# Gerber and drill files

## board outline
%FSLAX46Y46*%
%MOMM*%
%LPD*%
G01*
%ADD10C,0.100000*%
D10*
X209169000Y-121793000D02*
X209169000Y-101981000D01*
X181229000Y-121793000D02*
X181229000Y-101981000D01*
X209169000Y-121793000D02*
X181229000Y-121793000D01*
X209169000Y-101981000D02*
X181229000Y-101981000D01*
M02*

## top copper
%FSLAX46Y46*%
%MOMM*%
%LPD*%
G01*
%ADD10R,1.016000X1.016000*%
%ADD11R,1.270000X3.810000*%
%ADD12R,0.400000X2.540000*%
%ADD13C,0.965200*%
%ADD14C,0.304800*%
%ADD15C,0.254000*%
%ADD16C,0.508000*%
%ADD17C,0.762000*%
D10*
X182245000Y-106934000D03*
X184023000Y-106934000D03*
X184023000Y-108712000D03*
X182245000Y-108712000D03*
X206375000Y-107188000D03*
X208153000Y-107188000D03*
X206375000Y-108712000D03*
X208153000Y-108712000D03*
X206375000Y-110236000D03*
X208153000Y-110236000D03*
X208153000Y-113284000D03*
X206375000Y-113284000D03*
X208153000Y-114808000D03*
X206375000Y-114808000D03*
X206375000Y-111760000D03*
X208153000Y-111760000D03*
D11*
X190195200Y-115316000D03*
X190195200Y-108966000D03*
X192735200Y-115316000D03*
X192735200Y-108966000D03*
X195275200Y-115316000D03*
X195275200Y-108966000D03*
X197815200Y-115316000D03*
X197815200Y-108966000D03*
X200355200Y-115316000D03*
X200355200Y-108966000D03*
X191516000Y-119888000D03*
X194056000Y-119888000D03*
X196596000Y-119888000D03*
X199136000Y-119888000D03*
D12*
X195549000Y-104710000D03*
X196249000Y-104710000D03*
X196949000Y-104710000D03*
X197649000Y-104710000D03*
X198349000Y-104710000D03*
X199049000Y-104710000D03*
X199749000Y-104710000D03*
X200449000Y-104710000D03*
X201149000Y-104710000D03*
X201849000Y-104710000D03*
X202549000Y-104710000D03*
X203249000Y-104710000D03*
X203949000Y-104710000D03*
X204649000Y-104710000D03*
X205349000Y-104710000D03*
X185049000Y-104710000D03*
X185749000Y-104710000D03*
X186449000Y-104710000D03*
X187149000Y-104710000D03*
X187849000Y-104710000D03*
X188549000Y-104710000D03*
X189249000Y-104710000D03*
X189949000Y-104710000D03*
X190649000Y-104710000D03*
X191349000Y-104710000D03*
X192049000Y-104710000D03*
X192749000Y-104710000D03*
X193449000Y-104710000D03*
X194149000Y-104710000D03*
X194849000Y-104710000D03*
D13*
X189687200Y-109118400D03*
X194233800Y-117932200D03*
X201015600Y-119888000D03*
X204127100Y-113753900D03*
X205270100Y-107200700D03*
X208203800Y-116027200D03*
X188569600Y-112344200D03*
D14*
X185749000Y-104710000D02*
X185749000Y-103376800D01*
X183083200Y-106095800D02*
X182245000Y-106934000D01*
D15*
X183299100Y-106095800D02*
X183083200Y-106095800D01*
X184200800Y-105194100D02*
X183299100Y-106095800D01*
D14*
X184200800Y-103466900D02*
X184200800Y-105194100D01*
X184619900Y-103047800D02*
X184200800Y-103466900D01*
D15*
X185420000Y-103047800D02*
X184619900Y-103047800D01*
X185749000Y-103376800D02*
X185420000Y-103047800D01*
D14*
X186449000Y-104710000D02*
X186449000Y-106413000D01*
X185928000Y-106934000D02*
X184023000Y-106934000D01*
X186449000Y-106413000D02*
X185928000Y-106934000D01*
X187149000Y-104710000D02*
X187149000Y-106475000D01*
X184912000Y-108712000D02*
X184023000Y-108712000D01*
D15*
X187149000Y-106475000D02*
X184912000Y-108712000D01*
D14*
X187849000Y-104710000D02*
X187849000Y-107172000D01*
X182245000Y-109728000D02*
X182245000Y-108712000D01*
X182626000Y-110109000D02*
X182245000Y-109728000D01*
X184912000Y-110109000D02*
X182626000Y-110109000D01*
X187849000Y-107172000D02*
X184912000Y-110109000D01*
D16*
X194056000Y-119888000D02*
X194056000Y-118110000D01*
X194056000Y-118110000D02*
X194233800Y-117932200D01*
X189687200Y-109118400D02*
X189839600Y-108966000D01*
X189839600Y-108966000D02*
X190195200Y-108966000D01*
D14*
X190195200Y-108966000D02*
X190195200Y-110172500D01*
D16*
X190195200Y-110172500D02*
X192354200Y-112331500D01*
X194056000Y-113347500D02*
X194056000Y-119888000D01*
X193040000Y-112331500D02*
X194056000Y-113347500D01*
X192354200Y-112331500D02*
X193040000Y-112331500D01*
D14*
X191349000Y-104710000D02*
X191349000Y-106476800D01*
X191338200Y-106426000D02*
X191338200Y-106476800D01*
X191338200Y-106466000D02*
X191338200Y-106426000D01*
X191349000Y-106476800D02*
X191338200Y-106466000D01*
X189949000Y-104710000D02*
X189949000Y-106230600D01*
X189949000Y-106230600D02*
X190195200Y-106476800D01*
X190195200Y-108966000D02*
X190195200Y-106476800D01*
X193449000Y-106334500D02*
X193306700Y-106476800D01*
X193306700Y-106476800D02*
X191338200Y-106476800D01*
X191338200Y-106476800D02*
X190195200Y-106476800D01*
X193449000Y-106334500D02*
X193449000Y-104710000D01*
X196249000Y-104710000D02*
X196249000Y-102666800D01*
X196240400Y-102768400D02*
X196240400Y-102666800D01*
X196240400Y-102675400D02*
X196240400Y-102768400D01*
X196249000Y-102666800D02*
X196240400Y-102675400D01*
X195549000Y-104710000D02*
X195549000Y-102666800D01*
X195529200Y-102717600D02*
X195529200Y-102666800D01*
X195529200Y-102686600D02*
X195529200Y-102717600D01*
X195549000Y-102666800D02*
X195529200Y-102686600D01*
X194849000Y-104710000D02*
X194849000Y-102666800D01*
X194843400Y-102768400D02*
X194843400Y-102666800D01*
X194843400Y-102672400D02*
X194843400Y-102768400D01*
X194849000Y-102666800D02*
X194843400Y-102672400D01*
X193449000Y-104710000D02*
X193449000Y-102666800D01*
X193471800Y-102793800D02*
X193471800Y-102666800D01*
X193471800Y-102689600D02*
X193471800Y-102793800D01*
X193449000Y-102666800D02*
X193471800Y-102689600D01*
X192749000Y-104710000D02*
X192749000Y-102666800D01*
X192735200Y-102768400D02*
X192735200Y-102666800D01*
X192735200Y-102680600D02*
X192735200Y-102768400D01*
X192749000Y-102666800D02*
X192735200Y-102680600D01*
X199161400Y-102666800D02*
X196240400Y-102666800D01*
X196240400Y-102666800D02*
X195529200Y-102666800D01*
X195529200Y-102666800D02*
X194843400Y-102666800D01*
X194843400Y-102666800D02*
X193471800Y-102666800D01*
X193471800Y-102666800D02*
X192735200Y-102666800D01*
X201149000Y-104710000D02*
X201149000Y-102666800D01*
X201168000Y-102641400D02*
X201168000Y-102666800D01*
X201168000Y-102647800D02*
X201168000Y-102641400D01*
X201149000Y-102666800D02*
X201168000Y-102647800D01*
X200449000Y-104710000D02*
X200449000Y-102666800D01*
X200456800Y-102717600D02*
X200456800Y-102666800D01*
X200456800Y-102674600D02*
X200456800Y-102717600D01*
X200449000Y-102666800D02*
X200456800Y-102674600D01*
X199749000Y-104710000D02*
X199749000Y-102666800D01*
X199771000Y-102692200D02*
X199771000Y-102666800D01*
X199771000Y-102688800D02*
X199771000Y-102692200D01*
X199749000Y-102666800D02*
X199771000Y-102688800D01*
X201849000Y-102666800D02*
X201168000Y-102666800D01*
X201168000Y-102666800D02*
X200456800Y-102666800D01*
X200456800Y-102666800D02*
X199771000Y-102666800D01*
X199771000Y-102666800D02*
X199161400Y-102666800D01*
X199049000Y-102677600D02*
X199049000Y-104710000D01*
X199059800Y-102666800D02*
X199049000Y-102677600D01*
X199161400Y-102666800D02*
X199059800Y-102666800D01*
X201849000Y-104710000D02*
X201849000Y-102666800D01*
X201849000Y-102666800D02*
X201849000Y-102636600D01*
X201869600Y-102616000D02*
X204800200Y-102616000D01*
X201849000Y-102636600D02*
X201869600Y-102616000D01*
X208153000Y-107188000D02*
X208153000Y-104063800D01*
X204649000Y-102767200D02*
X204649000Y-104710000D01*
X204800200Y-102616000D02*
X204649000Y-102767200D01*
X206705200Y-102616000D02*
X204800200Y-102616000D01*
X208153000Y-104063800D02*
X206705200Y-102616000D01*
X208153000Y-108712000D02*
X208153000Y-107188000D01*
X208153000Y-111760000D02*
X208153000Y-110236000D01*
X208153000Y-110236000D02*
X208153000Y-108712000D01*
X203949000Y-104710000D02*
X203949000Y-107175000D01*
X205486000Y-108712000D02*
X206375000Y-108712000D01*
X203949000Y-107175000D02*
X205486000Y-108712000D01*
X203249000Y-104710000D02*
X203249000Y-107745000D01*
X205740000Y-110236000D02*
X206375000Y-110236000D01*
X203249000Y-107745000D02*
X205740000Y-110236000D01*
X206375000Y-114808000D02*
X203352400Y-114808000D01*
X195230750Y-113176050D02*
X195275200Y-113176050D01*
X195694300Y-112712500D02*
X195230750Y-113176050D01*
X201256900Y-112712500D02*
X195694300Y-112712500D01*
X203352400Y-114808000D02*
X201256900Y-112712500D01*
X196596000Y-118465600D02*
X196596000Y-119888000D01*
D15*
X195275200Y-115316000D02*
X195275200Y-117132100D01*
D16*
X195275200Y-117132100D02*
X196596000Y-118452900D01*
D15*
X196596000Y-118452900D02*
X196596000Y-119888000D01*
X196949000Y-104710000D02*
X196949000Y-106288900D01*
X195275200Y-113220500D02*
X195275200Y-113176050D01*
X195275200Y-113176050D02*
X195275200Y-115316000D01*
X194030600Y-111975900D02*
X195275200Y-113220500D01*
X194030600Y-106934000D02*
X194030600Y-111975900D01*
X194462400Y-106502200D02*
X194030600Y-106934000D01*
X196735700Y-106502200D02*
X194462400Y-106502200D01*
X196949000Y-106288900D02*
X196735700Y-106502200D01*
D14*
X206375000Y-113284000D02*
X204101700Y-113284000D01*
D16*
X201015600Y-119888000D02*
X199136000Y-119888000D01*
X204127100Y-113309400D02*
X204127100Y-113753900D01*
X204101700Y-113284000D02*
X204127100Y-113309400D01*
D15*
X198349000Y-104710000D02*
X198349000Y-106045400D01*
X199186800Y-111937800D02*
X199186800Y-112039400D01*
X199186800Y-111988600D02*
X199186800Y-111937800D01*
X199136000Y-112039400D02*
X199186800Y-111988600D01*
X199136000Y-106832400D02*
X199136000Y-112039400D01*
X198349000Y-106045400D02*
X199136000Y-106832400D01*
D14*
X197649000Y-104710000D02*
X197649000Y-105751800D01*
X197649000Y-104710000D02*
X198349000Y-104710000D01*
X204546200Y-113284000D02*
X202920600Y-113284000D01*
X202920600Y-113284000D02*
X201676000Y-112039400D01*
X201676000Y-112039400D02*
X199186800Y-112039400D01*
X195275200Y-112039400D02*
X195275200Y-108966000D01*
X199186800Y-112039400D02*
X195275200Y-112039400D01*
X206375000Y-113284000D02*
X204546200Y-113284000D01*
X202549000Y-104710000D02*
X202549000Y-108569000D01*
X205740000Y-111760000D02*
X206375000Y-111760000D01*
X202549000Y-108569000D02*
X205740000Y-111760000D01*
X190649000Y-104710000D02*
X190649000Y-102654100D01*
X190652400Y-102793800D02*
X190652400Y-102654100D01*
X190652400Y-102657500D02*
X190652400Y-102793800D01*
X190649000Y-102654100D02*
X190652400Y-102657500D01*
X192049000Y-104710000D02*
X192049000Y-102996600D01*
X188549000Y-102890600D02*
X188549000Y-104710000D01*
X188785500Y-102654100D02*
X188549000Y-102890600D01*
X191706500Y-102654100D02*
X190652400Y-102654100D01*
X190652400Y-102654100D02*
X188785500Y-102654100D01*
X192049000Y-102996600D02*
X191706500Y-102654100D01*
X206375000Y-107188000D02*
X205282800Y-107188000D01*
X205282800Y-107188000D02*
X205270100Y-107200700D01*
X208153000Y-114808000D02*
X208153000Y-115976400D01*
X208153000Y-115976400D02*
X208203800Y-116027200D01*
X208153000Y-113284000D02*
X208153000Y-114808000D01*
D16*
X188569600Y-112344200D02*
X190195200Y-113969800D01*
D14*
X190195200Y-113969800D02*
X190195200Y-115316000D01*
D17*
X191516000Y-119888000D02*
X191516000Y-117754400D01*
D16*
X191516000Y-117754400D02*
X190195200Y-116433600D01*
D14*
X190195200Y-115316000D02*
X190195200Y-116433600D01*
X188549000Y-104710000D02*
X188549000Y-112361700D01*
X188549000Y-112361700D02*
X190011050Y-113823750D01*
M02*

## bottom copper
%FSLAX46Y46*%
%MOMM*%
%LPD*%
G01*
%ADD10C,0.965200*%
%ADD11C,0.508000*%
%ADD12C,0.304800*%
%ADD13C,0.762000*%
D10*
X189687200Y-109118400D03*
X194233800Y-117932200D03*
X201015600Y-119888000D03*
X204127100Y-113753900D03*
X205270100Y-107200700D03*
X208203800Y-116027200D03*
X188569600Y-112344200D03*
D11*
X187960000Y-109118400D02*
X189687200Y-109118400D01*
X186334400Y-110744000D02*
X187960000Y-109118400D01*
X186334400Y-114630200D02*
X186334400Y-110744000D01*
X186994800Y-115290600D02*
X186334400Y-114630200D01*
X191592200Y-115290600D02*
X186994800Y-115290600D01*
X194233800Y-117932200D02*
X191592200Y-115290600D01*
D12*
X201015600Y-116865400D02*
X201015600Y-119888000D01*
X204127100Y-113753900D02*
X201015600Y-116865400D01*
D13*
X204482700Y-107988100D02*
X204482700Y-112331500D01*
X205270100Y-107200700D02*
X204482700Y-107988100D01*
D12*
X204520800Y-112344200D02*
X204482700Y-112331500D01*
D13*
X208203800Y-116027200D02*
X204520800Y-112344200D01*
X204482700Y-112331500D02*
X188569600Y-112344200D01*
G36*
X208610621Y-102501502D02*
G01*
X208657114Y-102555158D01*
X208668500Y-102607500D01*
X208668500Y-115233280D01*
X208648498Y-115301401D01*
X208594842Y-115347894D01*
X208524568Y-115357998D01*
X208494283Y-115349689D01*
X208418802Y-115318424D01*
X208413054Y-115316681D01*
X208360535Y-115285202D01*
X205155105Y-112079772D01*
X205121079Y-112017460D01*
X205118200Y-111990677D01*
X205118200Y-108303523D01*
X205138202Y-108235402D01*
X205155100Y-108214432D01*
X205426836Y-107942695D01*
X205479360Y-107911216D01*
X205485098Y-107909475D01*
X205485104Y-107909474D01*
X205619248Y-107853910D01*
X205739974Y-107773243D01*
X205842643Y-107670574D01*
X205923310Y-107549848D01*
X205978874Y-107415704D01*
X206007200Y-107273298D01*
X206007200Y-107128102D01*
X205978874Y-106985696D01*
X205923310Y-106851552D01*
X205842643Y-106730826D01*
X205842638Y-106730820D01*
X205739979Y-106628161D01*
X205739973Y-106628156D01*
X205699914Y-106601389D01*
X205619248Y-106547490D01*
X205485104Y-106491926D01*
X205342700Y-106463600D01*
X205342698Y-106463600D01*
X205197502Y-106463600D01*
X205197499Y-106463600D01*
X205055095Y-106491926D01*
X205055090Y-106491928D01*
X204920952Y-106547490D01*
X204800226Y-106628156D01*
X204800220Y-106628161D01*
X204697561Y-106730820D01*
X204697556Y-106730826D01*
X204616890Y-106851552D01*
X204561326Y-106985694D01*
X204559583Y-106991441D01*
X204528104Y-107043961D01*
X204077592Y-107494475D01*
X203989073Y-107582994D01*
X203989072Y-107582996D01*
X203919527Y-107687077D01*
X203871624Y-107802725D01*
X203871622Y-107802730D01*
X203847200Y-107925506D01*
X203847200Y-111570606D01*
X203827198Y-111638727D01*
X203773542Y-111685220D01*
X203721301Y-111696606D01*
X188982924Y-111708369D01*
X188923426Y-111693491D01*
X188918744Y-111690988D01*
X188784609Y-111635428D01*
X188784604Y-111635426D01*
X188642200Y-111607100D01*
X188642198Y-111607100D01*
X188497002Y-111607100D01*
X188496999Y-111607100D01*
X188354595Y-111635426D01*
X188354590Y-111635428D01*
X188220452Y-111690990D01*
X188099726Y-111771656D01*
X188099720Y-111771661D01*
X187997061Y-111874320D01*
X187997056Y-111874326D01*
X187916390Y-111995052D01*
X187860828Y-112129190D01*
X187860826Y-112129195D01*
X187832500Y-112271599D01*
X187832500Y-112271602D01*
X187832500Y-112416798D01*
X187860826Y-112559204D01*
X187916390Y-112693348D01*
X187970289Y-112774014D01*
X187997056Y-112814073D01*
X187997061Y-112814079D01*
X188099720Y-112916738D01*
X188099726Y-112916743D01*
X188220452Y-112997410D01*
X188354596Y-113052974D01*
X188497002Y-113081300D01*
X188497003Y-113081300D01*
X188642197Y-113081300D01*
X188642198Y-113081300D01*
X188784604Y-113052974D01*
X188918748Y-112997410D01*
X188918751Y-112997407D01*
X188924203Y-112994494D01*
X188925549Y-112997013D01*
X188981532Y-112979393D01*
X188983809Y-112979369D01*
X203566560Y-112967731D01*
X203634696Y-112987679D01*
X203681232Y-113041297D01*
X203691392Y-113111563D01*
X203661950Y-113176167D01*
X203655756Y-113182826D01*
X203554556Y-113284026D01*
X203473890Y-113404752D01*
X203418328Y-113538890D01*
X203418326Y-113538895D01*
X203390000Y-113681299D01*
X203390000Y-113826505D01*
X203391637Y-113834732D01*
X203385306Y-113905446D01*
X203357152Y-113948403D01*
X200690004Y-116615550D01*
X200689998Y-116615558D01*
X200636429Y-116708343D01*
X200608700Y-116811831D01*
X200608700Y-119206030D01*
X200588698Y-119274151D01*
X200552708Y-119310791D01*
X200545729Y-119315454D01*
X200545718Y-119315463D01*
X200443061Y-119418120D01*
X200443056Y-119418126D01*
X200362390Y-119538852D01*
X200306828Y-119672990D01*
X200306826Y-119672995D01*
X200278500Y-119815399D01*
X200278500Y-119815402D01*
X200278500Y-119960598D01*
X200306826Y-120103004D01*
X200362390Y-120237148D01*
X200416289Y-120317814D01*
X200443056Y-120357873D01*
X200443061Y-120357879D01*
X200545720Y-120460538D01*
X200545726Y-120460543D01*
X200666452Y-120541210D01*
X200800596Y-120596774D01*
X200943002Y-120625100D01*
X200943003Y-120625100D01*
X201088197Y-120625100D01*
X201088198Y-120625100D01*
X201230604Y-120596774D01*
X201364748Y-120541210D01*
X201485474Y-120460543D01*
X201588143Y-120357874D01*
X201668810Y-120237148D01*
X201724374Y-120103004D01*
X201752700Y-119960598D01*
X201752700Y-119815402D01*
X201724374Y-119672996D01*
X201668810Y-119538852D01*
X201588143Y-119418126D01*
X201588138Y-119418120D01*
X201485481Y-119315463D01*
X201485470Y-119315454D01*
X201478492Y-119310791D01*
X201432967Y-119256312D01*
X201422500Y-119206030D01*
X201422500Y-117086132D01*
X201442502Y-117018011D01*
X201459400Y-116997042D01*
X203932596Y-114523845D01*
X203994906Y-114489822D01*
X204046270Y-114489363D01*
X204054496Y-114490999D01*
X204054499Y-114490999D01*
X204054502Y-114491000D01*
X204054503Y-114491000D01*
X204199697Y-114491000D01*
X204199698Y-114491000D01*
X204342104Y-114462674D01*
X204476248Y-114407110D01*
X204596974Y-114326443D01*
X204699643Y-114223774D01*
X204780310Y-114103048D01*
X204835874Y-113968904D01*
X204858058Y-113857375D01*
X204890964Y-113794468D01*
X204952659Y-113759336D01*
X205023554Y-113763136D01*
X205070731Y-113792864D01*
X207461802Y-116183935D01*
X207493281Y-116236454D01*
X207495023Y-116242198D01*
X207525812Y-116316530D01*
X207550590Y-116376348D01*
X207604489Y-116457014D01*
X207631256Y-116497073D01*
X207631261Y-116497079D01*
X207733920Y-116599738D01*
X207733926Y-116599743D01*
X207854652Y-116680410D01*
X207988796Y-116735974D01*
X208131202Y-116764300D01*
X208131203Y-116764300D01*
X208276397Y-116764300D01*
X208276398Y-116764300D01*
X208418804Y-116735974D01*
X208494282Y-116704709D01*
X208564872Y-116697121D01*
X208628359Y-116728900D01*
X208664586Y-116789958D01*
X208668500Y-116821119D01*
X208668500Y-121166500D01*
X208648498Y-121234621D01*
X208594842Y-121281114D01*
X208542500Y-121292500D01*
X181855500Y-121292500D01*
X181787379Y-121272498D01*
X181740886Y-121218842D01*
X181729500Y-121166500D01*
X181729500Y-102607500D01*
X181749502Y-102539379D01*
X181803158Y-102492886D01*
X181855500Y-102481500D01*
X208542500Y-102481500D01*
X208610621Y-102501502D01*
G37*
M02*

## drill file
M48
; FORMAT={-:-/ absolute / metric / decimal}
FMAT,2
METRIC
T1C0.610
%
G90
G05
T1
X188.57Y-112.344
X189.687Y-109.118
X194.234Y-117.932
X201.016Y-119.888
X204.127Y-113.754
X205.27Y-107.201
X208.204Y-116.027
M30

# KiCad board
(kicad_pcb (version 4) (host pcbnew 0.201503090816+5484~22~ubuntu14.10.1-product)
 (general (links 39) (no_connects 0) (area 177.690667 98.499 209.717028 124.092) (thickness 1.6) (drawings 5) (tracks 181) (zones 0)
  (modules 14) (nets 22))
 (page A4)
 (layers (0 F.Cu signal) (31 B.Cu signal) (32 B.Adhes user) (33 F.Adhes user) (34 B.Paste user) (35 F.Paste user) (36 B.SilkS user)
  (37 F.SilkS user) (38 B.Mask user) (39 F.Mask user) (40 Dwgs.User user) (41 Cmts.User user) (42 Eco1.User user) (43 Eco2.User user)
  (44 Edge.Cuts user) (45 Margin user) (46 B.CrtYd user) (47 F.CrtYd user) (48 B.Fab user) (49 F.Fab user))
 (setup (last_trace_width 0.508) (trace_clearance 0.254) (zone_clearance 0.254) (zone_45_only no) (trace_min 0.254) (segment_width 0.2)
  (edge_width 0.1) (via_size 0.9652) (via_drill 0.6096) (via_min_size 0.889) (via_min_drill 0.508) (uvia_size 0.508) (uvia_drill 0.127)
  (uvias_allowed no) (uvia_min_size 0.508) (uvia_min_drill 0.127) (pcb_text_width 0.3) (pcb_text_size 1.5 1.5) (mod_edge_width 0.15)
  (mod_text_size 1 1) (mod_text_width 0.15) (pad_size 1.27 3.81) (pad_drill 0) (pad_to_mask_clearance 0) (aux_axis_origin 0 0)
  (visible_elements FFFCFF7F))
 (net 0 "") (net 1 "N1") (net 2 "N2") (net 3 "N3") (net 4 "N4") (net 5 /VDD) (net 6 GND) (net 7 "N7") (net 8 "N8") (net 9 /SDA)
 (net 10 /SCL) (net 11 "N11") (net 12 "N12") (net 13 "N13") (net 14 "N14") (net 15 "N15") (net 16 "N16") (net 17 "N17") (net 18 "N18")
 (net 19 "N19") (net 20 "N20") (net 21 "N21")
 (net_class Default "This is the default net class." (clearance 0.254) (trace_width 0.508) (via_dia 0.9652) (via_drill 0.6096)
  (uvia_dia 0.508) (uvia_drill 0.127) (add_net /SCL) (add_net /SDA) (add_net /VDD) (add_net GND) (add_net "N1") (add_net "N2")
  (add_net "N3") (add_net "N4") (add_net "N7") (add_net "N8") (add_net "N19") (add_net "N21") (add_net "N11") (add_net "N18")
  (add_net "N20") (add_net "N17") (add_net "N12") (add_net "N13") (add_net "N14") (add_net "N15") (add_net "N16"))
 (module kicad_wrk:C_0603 (layer F.Cu) (at 183.134 106.934)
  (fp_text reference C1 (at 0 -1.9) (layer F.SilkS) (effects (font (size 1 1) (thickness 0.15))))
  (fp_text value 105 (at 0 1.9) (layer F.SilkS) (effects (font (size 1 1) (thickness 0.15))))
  (pad 1 smd rect (at -0.889 0) (size 1.016 1.016) (layers F.Cu F.Paste F.Mask) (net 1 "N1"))
  (pad 2 smd rect (at 0.889 0) (size 1.016 1.016) (layers F.Cu F.Paste F.Mask) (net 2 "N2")))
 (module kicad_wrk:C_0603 (layer F.Cu) (at 183.134 108.712 180)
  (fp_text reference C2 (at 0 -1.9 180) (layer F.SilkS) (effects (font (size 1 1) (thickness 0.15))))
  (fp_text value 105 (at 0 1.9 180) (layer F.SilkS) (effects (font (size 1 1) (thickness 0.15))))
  (pad 1 smd rect (at -0.889 0 180) (size 1.016 1.016) (layers F.Cu F.Paste F.Mask) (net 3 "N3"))
  (pad 2 smd rect (at 0.889 0 180) (size 1.016 1.016) (layers F.Cu F.Paste F.Mask) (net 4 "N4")))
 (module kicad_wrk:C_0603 (layer F.Cu) (at 207.264 107.188)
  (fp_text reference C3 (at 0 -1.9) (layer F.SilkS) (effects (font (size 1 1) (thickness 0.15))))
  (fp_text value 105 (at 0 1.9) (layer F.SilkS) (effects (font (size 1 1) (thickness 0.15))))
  (pad 1 smd rect (at -0.889 0) (size 1.016 1.016) (layers F.Cu F.Paste F.Mask) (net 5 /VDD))
  (pad 2 smd rect (at 0.889 0) (size 1.016 1.016) (layers F.Cu F.Paste F.Mask) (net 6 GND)))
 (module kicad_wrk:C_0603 (layer F.Cu) (at 207.264 108.712)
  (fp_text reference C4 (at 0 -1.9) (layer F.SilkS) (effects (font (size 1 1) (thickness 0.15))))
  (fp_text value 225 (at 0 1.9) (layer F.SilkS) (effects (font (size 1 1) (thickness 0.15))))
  (pad 1 smd rect (at -0.889 0) (size 1.016 1.016) (layers F.Cu F.Paste F.Mask) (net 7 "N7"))
  (pad 2 smd rect (at 0.889 0) (size 1.016 1.016) (layers F.Cu F.Paste F.Mask) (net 6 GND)))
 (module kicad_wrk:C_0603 (layer F.Cu) (at 207.264 110.236)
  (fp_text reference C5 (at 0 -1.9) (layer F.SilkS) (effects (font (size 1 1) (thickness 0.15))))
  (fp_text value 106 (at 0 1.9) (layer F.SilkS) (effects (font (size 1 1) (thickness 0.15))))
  (pad 1 smd rect (at -0.889 0) (size 1.016 1.016) (layers F.Cu F.Paste F.Mask) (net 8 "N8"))
  (pad 2 smd rect (at 0.889 0) (size 1.016 1.016) (layers F.Cu F.Paste F.Mask) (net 6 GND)))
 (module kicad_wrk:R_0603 (layer F.Cu) (at 207.264 113.284 180)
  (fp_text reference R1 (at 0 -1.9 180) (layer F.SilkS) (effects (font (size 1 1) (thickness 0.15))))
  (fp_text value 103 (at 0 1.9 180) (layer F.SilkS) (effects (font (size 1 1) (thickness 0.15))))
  (pad 1 smd rect (at -0.889 0 180) (size 1.016 1.016) (layers F.Cu F.Paste F.Mask) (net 5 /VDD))
  (pad 2 smd rect (at 0.889 0 180) (size 1.016 1.016) (layers F.Cu F.Paste F.Mask) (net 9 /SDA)))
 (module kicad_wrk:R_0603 (layer F.Cu) (at 207.264 114.808 180)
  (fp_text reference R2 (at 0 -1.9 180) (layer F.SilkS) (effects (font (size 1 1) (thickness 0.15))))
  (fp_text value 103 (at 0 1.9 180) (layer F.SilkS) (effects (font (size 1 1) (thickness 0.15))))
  (pad 1 smd rect (at -0.889 0 180) (size 1.016 1.016) (layers F.Cu F.Paste F.Mask) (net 5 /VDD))
  (pad 2 smd rect (at 0.889 0 180) (size 1.016 1.016) (layers F.Cu F.Paste F.Mask) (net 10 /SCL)))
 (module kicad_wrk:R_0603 (layer F.Cu) (at 207.264 111.76)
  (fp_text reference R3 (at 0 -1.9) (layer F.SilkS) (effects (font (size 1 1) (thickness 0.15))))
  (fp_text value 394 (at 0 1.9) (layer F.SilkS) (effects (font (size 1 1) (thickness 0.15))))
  (pad 1 smd rect (at -0.889 0) (size 1.016 1.016) (layers F.Cu F.Paste F.Mask) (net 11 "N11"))
  (pad 2 smd rect (at 0.889 0) (size 1.016 1.016) (layers F.Cu F.Paste F.Mask) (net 6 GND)))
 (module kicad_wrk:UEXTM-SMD (layer F.Cu) (at 195.2752 112.141 180)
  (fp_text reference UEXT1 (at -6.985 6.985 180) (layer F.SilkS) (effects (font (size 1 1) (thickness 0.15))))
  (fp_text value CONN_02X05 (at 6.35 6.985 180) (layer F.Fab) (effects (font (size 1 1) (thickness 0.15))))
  (pad 1 smd rect (at 5.08 -3.175 180) (size 1.27 3.81) (layers F.Cu F.Paste F.Mask) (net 5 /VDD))
  (pad 2 smd rect (at 5.08 3.175 180) (size 1.27 3.81) (layers F.Cu F.Paste F.Mask) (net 6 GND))
  (pad 3 smd rect (at 2.54 -3.175 180) (size 1.27 3.81) (layers F.Cu F.Paste F.Mask) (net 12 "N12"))
  (pad 4 smd rect (at 2.54 3.175 180) (size 1.27 3.81) (layers F.Cu F.Paste F.Mask) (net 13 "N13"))
  (pad 5 smd rect (at 0 -3.175 180) (size 1.27 3.81) (layers F.Cu F.Paste F.Mask) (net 10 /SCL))
  (pad 6 smd rect (at 0 3.175 180) (size 1.27 3.81) (layers F.Cu F.Paste F.Mask) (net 9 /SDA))
  (pad 7 smd rect (at -2.54 -3.175 180) (size 1.27 3.81) (layers F.Cu F.Paste F.Mask) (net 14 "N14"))
  (pad 8 smd rect (at -2.54 3.175 180) (size 1.27 3.81) (layers F.Cu F.Paste F.Mask) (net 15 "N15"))
  (pad 9 smd rect (at -5.08 -3.175 180) (size 1.27 3.81) (layers F.Cu F.Paste F.Mask) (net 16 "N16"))
  (pad 10 smd rect (at -5.08 3.175 180) (size 1.27 3.81) (layers F.Cu F.Paste F.Mask) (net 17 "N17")))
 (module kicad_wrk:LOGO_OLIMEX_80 (layer F.Cu) (at 205.5876 118.6942)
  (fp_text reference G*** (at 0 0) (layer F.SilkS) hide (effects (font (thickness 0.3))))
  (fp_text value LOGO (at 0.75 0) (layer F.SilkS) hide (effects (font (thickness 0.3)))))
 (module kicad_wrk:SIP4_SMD (layer F.Cu) (at 195.326 119.888)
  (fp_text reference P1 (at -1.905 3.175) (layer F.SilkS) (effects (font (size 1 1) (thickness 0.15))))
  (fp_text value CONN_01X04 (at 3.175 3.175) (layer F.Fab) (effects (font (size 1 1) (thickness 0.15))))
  (pad 1 smd rect (at -3.81 0) (size 1.27 3.81) (layers F.Cu F.Mask) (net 5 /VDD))
  (pad 2 smd rect (at -1.27 0) (size 1.27 3.81) (layers F.Cu F.Mask) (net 6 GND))
  (pad 3 smd rect (at 1.27 0) (size 1.27 3.81) (layers F.Cu F.Mask) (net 10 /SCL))
  (pad 4 smd rect (at 3.81 0) (size 1.27 3.81) (layers F.Cu F.Mask) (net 9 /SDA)))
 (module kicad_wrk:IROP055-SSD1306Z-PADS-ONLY (layer F.Cu) (at 195.199 105.41)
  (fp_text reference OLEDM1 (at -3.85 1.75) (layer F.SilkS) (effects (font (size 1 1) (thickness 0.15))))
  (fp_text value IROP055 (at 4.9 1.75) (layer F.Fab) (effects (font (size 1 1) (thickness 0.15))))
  (pad 16 smd rect (at 0.35 -0.7) (size 0.4 2.54) (layers F.Cu F.Paste F.Mask) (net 6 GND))
  (pad 17 smd rect (at 1.05 -0.7) (size 0.4 2.54) (layers F.Cu F.Paste F.Mask) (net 6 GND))
  (pad 18 smd rect (at 1.75 -0.7) (size 0.4 2.54) (layers F.Cu F.Paste F.Mask) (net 10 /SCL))
  (pad 19 smd rect (at 2.45 -0.7) (size 0.4 2.54) (layers F.Cu F.Paste F.Mask) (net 9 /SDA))
  (pad 20 smd rect (at 3.15 -0.7) (size 0.4 2.54) (layers F.Cu F.Paste F.Mask) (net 9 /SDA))
  (pad 21 smd rect (at 3.85 -0.7) (size 0.4 2.54) (layers F.Cu F.Paste F.Mask) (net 6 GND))
  (pad 22 smd rect (at 4.55 -0.7) (size 0.4 2.54) (layers F.Cu F.Paste F.Mask) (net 6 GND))
  (pad 23 smd rect (at 5.25 -0.7) (size 0.4 2.54) (layers F.Cu F.Paste F.Mask) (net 6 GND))
  (pad 24 smd rect (at 5.95 -0.7) (size 0.4 2.54) (layers F.Cu F.Paste F.Mask) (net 6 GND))
  (pad 25 smd rect (at 6.65 -0.7) (size 0.4 2.54) (layers F.Cu F.Paste F.Mask) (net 6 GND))
  (pad 26 smd rect (at 7.35 -0.7) (size 0.4 2.54) (layers F.Cu F.Paste F.Mask) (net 11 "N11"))
  (pad 27 smd rect (at 8.05 -0.7) (size 0.4 2.54) (layers F.Cu F.Paste F.Mask) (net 8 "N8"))
  (pad 28 smd rect (at 8.75 -0.7) (size 0.4 2.54) (layers F.Cu F.Paste F.Mask) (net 7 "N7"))
  (pad 29 smd rect (at 9.45 -0.7) (size 0.4 2.54) (layers F.Cu F.Paste F.Mask) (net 6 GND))
  (pad 30 smd rect (at 10.15 -0.7) (size 0.4 2.54) (layers F.Cu F.Paste F.Mask) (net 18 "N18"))
  (pad 1 smd rect (at -10.15 -0.7) (size 0.4 2.54) (layers F.Cu F.Paste F.Mask) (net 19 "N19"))
  (pad 2 smd rect (at -9.45 -0.7) (size 0.4 2.54) (layers F.Cu F.Paste F.Mask) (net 1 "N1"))
  (pad 3 smd rect (at -8.75 -0.7) (size 0.4 2.54) (layers F.Cu F.Paste F.Mask) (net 2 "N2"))
  (pad 4 smd rect (at -8.05 -0.7) (size 0.4 2.54) (layers F.Cu F.Paste F.Mask) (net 3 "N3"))
  (pad 5 smd rect (at -7.35 -0.7) (size 0.4 2.54) (layers F.Cu F.Paste F.Mask) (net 4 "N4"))
  (pad 6 smd rect (at -6.65 -0.7) (size 0.4 2.54) (layers F.Cu F.Paste F.Mask) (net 5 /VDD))
  (pad 7 smd rect (at -5.95 -0.7) (size 0.4 2.54) (layers F.Cu F.Paste F.Mask) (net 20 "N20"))
  (pad 8 smd rect (at -5.25 -0.7) (size 0.4 2.54) (layers F.Cu F.Paste F.Mask) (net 6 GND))
  (pad 9 smd rect (at -4.55 -0.7) (size 0.4 2.54) (layers F.Cu F.Paste F.Mask) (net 5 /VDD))
  (pad 10 smd rect (at -3.85 -0.7) (size 0.4 2.54) (layers F.Cu F.Paste F.Mask) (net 6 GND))
  (pad 11 smd rect (at -3.15 -0.7) (size 0.4 2.54) (layers F.Cu F.Paste F.Mask) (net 5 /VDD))
  (pad 12 smd rect (at -2.45 -0.7) (size 0.4 2.54) (layers F.Cu F.Paste F.Mask) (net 6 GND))
  (pad 13 smd rect (at -1.75 -0.7) (size 0.4 2.54) (layers F.Cu F.Paste F.Mask) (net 6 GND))
  (pad 14 smd rect (at -1.05 -0.7) (size 0.4 2.54) (layers F.Cu F.Paste F.Mask) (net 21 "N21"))
  (pad 15 smd rect (at -0.35 -0.7) (size 0.4 2.54) (layers F.Cu F.Paste F.Mask) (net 6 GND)))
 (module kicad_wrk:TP (layer F.Cu) (at 182.753 103.378 180)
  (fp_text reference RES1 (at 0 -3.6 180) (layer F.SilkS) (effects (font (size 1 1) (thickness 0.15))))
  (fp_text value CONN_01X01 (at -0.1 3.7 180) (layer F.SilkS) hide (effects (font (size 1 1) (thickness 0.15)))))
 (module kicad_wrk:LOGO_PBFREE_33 (layer F.Cu) (at 183.6166 118.8466)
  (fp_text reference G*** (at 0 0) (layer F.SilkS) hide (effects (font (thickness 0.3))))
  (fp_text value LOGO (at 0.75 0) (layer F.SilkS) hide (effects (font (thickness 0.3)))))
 (gr_line (start 209.169 121.793) (end 209.169 101.981) (angle 90) (layer Edge.Cuts) (width 0.1))
 (gr_line (start 181.229 121.793) (end 181.229 101.981) (angle 90) (layer Edge.Cuts) (width 0.1))
 (gr_line (start 209.169 121.793) (end 181.229 121.793) (angle 90) (layer Edge.Cuts) (width 0.1))
 (gr_line (start 209.169 101.981) (end 181.229 101.981) (angle 90) (layer Edge.Cuts) (width 0.1))
 (segment (start 185.749 104.71) (end 185.749 103.3768) (width 0.3048) (layer F.Cu) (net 1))
 (segment (start 183.0832 106.0958) (end 182.245 106.934) (width 0.3048) (layer F.Cu) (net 1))
 (segment (start 183.2991 106.0958) (end 183.0832 106.0958) (width 0.254) (layer F.Cu) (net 1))
 (segment (start 184.2008 105.1941) (end 183.2991 106.0958) (width 0.254) (layer F.Cu) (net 1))
 (segment (start 184.2008 103.4669) (end 184.2008 105.1941) (width 0.3048) (layer F.Cu) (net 1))
 (segment (start 184.6199 103.0478) (end 184.2008 103.4669) (width 0.3048) (layer F.Cu) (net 1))
 (segment (start 185.42 103.0478) (end 184.6199 103.0478) (width 0.254) (layer F.Cu) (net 1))
 (segment (start 185.749 103.3768) (end 185.42 103.0478) (width 0.254) (layer F.Cu) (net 1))
 (segment (start 186.449 104.71) (end 186.449 106.413) (width 0.3048) (layer F.Cu) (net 2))
 (segment (start 185.928 106.934) (end 184.023 106.934) (width 0.3048) (layer F.Cu) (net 2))
 (segment (start 186.449 106.413) (end 185.928 106.934) (width 0.3048) (layer F.Cu) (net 2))
 (segment (start 187.149 104.71) (end 187.149 106.475) (width 0.3048) (layer F.Cu) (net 3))
 (segment (start 184.912 108.712) (end 184.023 108.712) (width 0.3048) (layer F.Cu) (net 3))
 (segment (start 187.149 106.475) (end 184.912 108.712) (width 0.254) (layer F.Cu) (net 3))
 (segment (start 187.849 104.71) (end 187.849 107.172) (width 0.3048) (layer F.Cu) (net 4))
 (segment (start 182.245 109.728) (end 182.245 108.712) (width 0.3048) (layer F.Cu) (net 4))
 (segment (start 182.626 110.109) (end 182.245 109.728) (width 0.3048) (layer F.Cu) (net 4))
 (segment (start 184.912 110.109) (end 182.626 110.109) (width 0.3048) (layer F.Cu) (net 4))
 (segment (start 187.849 107.172) (end 184.912 110.109) (width 0.3048) (layer F.Cu) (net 4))
 (segment (start 194.056 119.888) (end 194.056 118.11) (width 0.508) (layer F.Cu) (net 6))
 (segment (start 194.056 118.11) (end 194.2338 117.9322) (width 0.508) (layer F.Cu) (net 6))
 (segment (start 189.6872 109.1184) (end 189.8396 108.966) (width 0.508) (layer F.Cu) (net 6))
 (via (at 189.6872 109.1184) (size 0.9652) (layers F.Cu B.Cu) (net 6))
 (segment (start 187.96 109.1184) (end 189.6872 109.1184) (width 0.508) (layer B.Cu) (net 6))
 (segment (start 186.3344 110.744) (end 187.96 109.1184) (width 0.508) (layer B.Cu) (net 6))
 (segment (start 186.3344 114.6302) (end 186.3344 110.744) (width 0.508) (layer B.Cu) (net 6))
 (segment (start 186.9948 115.2906) (end 186.3344 114.6302) (width 0.508) (layer B.Cu) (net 6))
 (segment (start 191.5922 115.2906) (end 186.9948 115.2906) (width 0.508) (layer B.Cu) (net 6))
 (segment (start 194.2338 117.9322) (end 191.5922 115.2906) (width 0.508) (layer B.Cu) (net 6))
 (via (at 194.2338 117.9322) (size 0.9652) (layers F.Cu B.Cu) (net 6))
 (segment (start 189.8396 108.966) (end 190.1952 108.966) (width 0.508) (layer F.Cu) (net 6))
 (segment (start 190.1952 108.966) (end 190.1952 110.1725) (width 0.3048) (layer F.Cu) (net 6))
 (segment (start 190.1952 110.1725) (end 192.3542 112.3315) (width 0.508) (layer F.Cu) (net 6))
 (segment (start 194.056 113.3475) (end 194.056 119.888) (width 0.508) (layer F.Cu) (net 6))
 (segment (start 193.04 112.3315) (end 194.056 113.3475) (width 0.508) (layer F.Cu) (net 6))
 (segment (start 192.3542 112.3315) (end 193.04 112.3315) (width 0.508) (layer F.Cu) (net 6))
 (segment (start 191.349 104.71) (end 191.349 106.4768) (width 0.3048) (layer F.Cu) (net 6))
 (segment (start 191.3382 106.426) (end 191.3382 106.4768) (width 0.3048) (layer F.Cu) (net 6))
 (segment (start 191.3382 106.466) (end 191.3382 106.426) (width 0.3048) (layer F.Cu) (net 6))
 (segment (start 191.349 106.4768) (end 191.3382 106.466) (width 0.3048) (layer F.Cu) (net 6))
 (segment (start 189.949 104.71) (end 189.949 106.2306) (width 0.3048) (layer F.Cu) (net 6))
 (segment (start 189.949 106.2306) (end 190.1952 106.4768) (width 0.3048) (layer F.Cu) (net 6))
 (segment (start 190.1952 108.966) (end 190.1952 106.4768) (width 0.3048) (layer F.Cu) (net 6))
 (segment (start 193.449 106.3345) (end 193.3067 106.4768) (width 0.3048) (layer F.Cu) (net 6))
 (segment (start 193.3067 106.4768) (end 191.3382 106.4768) (width 0.3048) (layer F.Cu) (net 6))
 (segment (start 191.3382 106.4768) (end 190.1952 106.4768) (width 0.3048) (layer F.Cu) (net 6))
 (segment (start 193.449 106.3345) (end 193.449 104.71) (width 0.3048) (layer F.Cu) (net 6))
 (segment (start 196.249 104.71) (end 196.249 102.6668) (width 0.3048) (layer F.Cu) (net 6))
 (segment (start 196.2404 102.7684) (end 196.2404 102.6668) (width 0.3048) (layer F.Cu) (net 6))
 (segment (start 196.2404 102.6754) (end 196.2404 102.7684) (width 0.3048) (layer F.Cu) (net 6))
 (segment (start 196.249 102.6668) (end 196.2404 102.6754) (width 0.3048) (layer F.Cu) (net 6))
 (segment (start 195.549 104.71) (end 195.549 102.6668) (width 0.3048) (layer F.Cu) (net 6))
 (segment (start 195.5292 102.7176) (end 195.5292 102.6668) (width 0.3048) (layer F.Cu) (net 6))
 (segment (start 195.5292 102.6866) (end 195.5292 102.7176) (width 0.3048) (layer F.Cu) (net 6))
 (segment (start 195.549 102.6668) (end 195.5292 102.6866) (width 0.3048) (layer F.Cu) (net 6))
 (segment (start 194.849 104.71) (end 194.849 102.6668) (width 0.3048) (layer F.Cu) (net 6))
 (segment (start 194.8434 102.7684) (end 194.8434 102.6668) (width 0.3048) (layer F.Cu) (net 6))
 (segment (start 194.8434 102.6724) (end 194.8434 102.7684) (width 0.3048) (layer F.Cu) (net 6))
 (segment (start 194.849 102.6668) (end 194.8434 102.6724) (width 0.3048) (layer F.Cu) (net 6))
 (segment (start 193.449 104.71) (end 193.449 102.6668) (width 0.3048) (layer F.Cu) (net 6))
 (segment (start 193.4718 102.7938) (end 193.4718 102.6668) (width 0.3048) (layer F.Cu) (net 6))
 (segment (start 193.4718 102.6896) (end 193.4718 102.7938) (width 0.3048) (layer F.Cu) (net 6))
 (segment (start 193.449 102.6668) (end 193.4718 102.6896) (width 0.3048) (layer F.Cu) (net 6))
 (segment (start 192.749 104.71) (end 192.749 102.6668) (width 0.3048) (layer F.Cu) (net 6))
 (segment (start 192.7352 102.7684) (end 192.7352 102.6668) (width 0.3048) (layer F.Cu) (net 6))
 (segment (start 192.7352 102.6806) (end 192.7352 102.7684) (width 0.3048) (layer F.Cu) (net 6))
 (segment (start 192.749 102.6668) (end 192.7352 102.6806) (width 0.3048) (layer F.Cu) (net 6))
 (segment (start 199.1614 102.6668) (end 196.2404 102.6668) (width 0.3048) (layer F.Cu) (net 6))
 (segment (start 196.2404 102.6668) (end 195.5292 102.6668) (width 0.3048) (layer F.Cu) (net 6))
 (segment (start 195.5292 102.6668) (end 194.8434 102.6668) (width 0.3048) (layer F.Cu) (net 6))
 (segment (start 194.8434 102.6668) (end 193.4718 102.6668) (width 0.3048) (layer F.Cu) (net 6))
 (segment (start 193.4718 102.6668) (end 192.7352 102.6668) (width 0.3048) (layer F.Cu) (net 6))
 (segment (start 201.149 104.71) (end 201.149 102.6668) (width 0.3048) (layer F.Cu) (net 6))
 (segment (start 201.168 102.6414) (end 201.168 102.6668) (width 0.3048) (layer F.Cu) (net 6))
 (segment (start 201.168 102.6478) (end 201.168 102.6414) (width 0.3048) (layer F.Cu) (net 6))
 (segment (start 201.149 102.6668) (end 201.168 102.6478) (width 0.3048) (layer F.Cu) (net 6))
 (segment (start 200.449 104.71) (end 200.449 102.6668) (width 0.3048) (layer F.Cu) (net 6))
 (segment (start 200.4568 102.7176) (end 200.4568 102.6668) (width 0.3048) (layer F.Cu) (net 6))
 (segment (start 200.4568 102.6746) (end 200.4568 102.7176) (width 0.3048) (layer F.Cu) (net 6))
 (segment (start 200.449 102.6668) (end 200.4568 102.6746) (width 0.3048) (layer F.Cu) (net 6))
 (segment (start 199.749 104.71) (end 199.749 102.6668) (width 0.3048) (layer F.Cu) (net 6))
 (segment (start 199.771 102.6922) (end 199.771 102.6668) (width 0.3048) (layer F.Cu) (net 6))
 (segment (start 199.771 102.6888) (end 199.771 102.6922) (width 0.3048) (layer F.Cu) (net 6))
 (segment (start 199.749 102.6668) (end 199.771 102.6888) (width 0.3048) (layer F.Cu) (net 6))
 (segment (start 201.849 102.6668) (end 201.168 102.6668) (width 0.3048) (layer F.Cu) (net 6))
 (segment (start 201.168 102.6668) (end 200.4568 102.6668) (width 0.3048) (layer F.Cu) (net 6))
 (segment (start 200.4568 102.6668) (end 199.771 102.6668) (width 0.3048) (layer F.Cu) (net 6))
 (segment (start 199.771 102.6668) (end 199.1614 102.6668) (width 0.3048) (layer F.Cu) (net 6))
 (segment (start 199.049 102.6776) (end 199.049 104.71) (width 0.3048) (layer F.Cu) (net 6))
 (segment (start 199.0598 102.6668) (end 199.049 102.6776) (width 0.3048) (layer F.Cu) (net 6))
 (segment (start 199.1614 102.6668) (end 199.0598 102.6668) (width 0.3048) (layer F.Cu) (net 6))
 (segment (start 201.849 104.71) (end 201.849 102.6668) (width 0.3048) (layer F.Cu) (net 6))
 (segment (start 201.849 102.6668) (end 201.849 102.6366) (width 0.3048) (layer F.Cu) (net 6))
 (segment (start 201.8696 102.616) (end 204.8002 102.616) (width 0.3048) (layer F.Cu) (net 6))
 (segment (start 201.849 102.6366) (end 201.8696 102.616) (width 0.3048) (layer F.Cu) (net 6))
 (segment (start 208.153 107.188) (end 208.153 104.0638) (width 0.3048) (layer F.Cu) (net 6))
 (segment (start 204.649 102.7672) (end 204.649 104.71) (width 0.3048) (layer F.Cu) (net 6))
 (segment (start 204.8002 102.616) (end 204.649 102.7672) (width 0.3048) (layer F.Cu) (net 6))
 (segment (start 206.7052 102.616) (end 204.8002 102.616) (width 0.3048) (layer F.Cu) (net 6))
 (segment (start 208.153 104.0638) (end 206.7052 102.616) (width 0.3048) (layer F.Cu) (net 6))
 (segment (start 208.153 108.712) (end 208.153 107.188) (width 0.3048) (layer F.Cu) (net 6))
 (segment (start 208.153 111.76) (end 208.153 110.236) (width 0.3048) (layer F.Cu) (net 6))
 (segment (start 208.153 110.236) (end 208.153 108.712) (width 0.3048) (layer F.Cu) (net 6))
 (segment (start 203.949 104.71) (end 203.949 107.175) (width 0.3048) (layer F.Cu) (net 7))
 (segment (start 205.486 108.712) (end 206.375 108.712) (width 0.3048) (layer F.Cu) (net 7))
 (segment (start 203.949 107.175) (end 205.486 108.712) (width 0.3048) (layer F.Cu) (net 7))
 (segment (start 203.249 104.71) (end 203.249 107.745) (width 0.3048) (layer F.Cu) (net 8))
 (segment (start 205.74 110.236) (end 206.375 110.236) (width 0.3048) (layer F.Cu) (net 8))
 (segment (start 203.249 107.745) (end 205.74 110.236) (width 0.3048) (layer F.Cu) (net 8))
 (segment (start 206.375 114.808) (end 203.3524 114.808) (width 0.3048) (layer F.Cu) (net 10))
 (segment (start 195.23075 113.17605) (end 195.2752 113.17605) (width 0.3048) (layer F.Cu) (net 10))
 (segment (start 195.6943 112.7125) (end 195.23075 113.17605) (width 0.3048) (layer F.Cu) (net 10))
 (segment (start 201.2569 112.7125) (end 195.6943 112.7125) (width 0.3048) (layer F.Cu) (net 10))
 (segment (start 203.3524 114.808) (end 201.2569 112.7125) (width 0.3048) (layer F.Cu) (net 10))
 (segment (start 196.596 118.4656) (end 196.596 119.888) (width 0.3048) (layer F.Cu) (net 10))
 (segment (start 195.2752 115.316) (end 195.2752 117.1321) (width 0.254) (layer F.Cu) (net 10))
 (segment (start 195.2752 117.1321) (end 196.596 118.4529) (width 0.508) (layer F.Cu) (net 10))
 (segment (start 196.596 118.4529) (end 196.596 119.888) (width 0.254) (layer F.Cu) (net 10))
 (segment (start 196.949 104.71) (end 196.949 106.2889) (width 0.254) (layer F.Cu) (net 10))
 (segment (start 195.2752 113.2205) (end 195.2752 113.17605) (width 0.254) (layer F.Cu) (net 10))
 (segment (start 195.2752 113.17605) (end 195.2752 115.316) (width 0.254) (layer F.Cu) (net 10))
 (segment (start 194.0306 111.9759) (end 195.2752 113.2205) (width 0.254) (layer F.Cu) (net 10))
 (segment (start 194.0306 106.934) (end 194.0306 111.9759) (width 0.254) (layer F.Cu) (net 10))
 (segment (start 194.4624 106.5022) (end 194.0306 106.934) (width 0.254) (layer F.Cu) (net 10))
 (segment (start 196.7357 106.5022) (end 194.4624 106.5022) (width 0.254) (layer F.Cu) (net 10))
 (segment (start 196.949 106.2889) (end 196.7357 106.5022) (width 0.254) (layer F.Cu) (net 10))
 (segment (start 206.375 113.284) (end 204.1017 113.284) (width 0.3048) (layer F.Cu) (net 9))
 (segment (start 201.0156 119.888) (end 199.136 119.888) (width 0.508) (layer F.Cu) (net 9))
 (via (at 201.0156 119.888) (size 0.9652) (layers F.Cu B.Cu) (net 9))
 (segment (start 201.0156 116.8654) (end 201.0156 119.888) (width 0.3048) (layer B.Cu) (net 9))
 (segment (start 204.1271 113.7539) (end 201.0156 116.8654) (width 0.3048) (layer B.Cu) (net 9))
 (via (at 204.1271 113.7539) (size 0.9652) (layers F.Cu B.Cu) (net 9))
 (segment (start 204.1271 113.3094) (end 204.1271 113.7539) (width 0.508) (layer F.Cu) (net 9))
 (segment (start 204.1017 113.284) (end 204.1271 113.3094) (width 0.508) (layer F.Cu) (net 9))
 (segment (start 198.349 104.71) (end 198.349 106.0454) (width 0.254) (layer F.Cu) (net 9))
 (segment (start 199.1868 111.9378) (end 199.1868 112.0394) (width 0.254) (layer F.Cu) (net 9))
 (segment (start 199.1868 111.9886) (end 199.1868 111.9378) (width 0.254) (layer F.Cu) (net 9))
 (segment (start 199.136 112.0394) (end 199.1868 111.9886) (width 0.254) (layer F.Cu) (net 9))
 (segment (start 199.136 106.8324) (end 199.136 112.0394) (width 0.254) (layer F.Cu) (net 9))
 (segment (start 198.349 106.0454) (end 199.136 106.8324) (width 0.254) (layer F.Cu) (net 9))
 (segment (start 197.649 104.71) (end 197.649 105.7518) (width 0.3048) (layer F.Cu) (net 9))
 (segment (start 197.649 104.71) (end 198.349 104.71) (width 0.3048) (layer F.Cu) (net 9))
 (segment (start 204.5462 113.284) (end 202.9206 113.284) (width 0.3048) (layer F.Cu) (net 9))
 (segment (start 202.9206 113.284) (end 201.676 112.0394) (width 0.3048) (layer F.Cu) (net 9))
 (segment (start 201.676 112.0394) (end 199.1868 112.0394) (width 0.3048) (layer F.Cu) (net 9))
 (segment (start 195.2752 112.0394) (end 195.2752 108.966) (width 0.3048) (layer F.Cu) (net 9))
 (segment (start 199.1868 112.0394) (end 195.2752 112.0394) (width 0.3048) (layer F.Cu) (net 9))
 (segment (start 206.375 113.284) (end 204.5462 113.284) (width 0.3048) (layer F.Cu) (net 9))
 (segment (start 202.549 104.71) (end 202.549 108.569) (width 0.3048) (layer F.Cu) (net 11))
 (segment (start 205.74 111.76) (end 206.375 111.76) (width 0.3048) (layer F.Cu) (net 11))
 (segment (start 202.549 108.569) (end 205.74 111.76) (width 0.3048) (layer F.Cu) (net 11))
 (segment (start 190.649 104.71) (end 190.649 102.6541) (width 0.3048) (layer F.Cu) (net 5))
 (segment (start 190.6524 102.7938) (end 190.6524 102.6541) (width 0.3048) (layer F.Cu) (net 5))
 (segment (start 190.6524 102.6575) (end 190.6524 102.7938) (width 0.3048) (layer F.Cu) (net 5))
 (segment (start 190.649 102.6541) (end 190.6524 102.6575) (width 0.3048) (layer F.Cu) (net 5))
 (segment (start 192.049 104.71) (end 192.049 102.9966) (width 0.3048) (layer F.Cu) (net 5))
 (segment (start 188.549 102.8906) (end 188.549 104.71) (width 0.3048) (layer F.Cu) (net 5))
 (segment (start 188.7855 102.6541) (end 188.549 102.8906) (width 0.3048) (layer F.Cu) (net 5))
 (segment (start 191.7065 102.6541) (end 190.6524 102.6541) (width 0.3048) (layer F.Cu) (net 5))
 (segment (start 190.6524 102.6541) (end 188.7855 102.6541) (width 0.3048) (layer F.Cu) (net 5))
 (segment (start 192.049 102.9966) (end 191.7065 102.6541) (width 0.3048) (layer F.Cu) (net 5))
 (segment (start 206.375 107.188) (end 205.2828 107.188) (width 0.3048) (layer F.Cu) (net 5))
 (segment (start 204.4827 107.9881) (end 204.4827 112.3315) (width 0.762) (layer B.Cu) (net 5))
 (segment (start 205.2701 107.2007) (end 204.4827 107.9881) (width 0.762) (layer B.Cu) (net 5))
 (via (at 205.2701 107.2007) (size 0.9652) (layers F.Cu B.Cu) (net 5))
 (segment (start 205.2828 107.188) (end 205.2701 107.2007) (width 0.3048) (layer F.Cu) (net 5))
 (segment (start 208.153 114.808) (end 208.153 115.9764) (width 0.3048) (layer F.Cu) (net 5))
 (segment (start 204.5208 112.3442) (end 204.4827 112.3315) (width 0.3048) (layer B.Cu) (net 5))
 (segment (start 208.2038 116.0272) (end 204.5208 112.3442) (width 0.762) (layer B.Cu) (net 5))
 (via (at 208.2038 116.0272) (size 0.9652) (layers F.Cu B.Cu) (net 5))
 (segment (start 208.153 115.9764) (end 208.2038 116.0272) (width 0.3048) (layer F.Cu) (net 5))
 (segment (start 208.153 113.284) (end 208.153 114.808) (width 0.3048) (layer F.Cu) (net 5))
 (segment (start 188.5696 112.3442) (end 190.1952 113.9698) (width 0.508) (layer F.Cu) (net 5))
 (segment (start 204.4827 112.3315) (end 188.5696 112.3442) (width 0.762) (layer B.Cu) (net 5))
 (via (at 188.5696 112.3442) (size 0.9652) (layers F.Cu B.Cu) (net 5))
 (segment (start 190.1952 113.9698) (end 190.1952 115.316) (width 0.3048) (layer F.Cu) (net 5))
 (segment (start 191.516 119.888) (end 191.516 117.7544) (width 0.762) (layer F.Cu) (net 5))
 (segment (start 191.516 117.7544) (end 190.1952 116.4336) (width 0.508) (layer F.Cu) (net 5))
 (segment (start 190.1952 115.316) (end 190.1952 116.4336) (width 0.3048) (layer F.Cu) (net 5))
 (segment (start 188.549 104.71) (end 188.549 112.3617) (width 0.3048) (layer F.Cu) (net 5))
 (segment (start 188.549 112.3617) (end 190.01105 113.82375) (width 0.3048) (layer F.Cu) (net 5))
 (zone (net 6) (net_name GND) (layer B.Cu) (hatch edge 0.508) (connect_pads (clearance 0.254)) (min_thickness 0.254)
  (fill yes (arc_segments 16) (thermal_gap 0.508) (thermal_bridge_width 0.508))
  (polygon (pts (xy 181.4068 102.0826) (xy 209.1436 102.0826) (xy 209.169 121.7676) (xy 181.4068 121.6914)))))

